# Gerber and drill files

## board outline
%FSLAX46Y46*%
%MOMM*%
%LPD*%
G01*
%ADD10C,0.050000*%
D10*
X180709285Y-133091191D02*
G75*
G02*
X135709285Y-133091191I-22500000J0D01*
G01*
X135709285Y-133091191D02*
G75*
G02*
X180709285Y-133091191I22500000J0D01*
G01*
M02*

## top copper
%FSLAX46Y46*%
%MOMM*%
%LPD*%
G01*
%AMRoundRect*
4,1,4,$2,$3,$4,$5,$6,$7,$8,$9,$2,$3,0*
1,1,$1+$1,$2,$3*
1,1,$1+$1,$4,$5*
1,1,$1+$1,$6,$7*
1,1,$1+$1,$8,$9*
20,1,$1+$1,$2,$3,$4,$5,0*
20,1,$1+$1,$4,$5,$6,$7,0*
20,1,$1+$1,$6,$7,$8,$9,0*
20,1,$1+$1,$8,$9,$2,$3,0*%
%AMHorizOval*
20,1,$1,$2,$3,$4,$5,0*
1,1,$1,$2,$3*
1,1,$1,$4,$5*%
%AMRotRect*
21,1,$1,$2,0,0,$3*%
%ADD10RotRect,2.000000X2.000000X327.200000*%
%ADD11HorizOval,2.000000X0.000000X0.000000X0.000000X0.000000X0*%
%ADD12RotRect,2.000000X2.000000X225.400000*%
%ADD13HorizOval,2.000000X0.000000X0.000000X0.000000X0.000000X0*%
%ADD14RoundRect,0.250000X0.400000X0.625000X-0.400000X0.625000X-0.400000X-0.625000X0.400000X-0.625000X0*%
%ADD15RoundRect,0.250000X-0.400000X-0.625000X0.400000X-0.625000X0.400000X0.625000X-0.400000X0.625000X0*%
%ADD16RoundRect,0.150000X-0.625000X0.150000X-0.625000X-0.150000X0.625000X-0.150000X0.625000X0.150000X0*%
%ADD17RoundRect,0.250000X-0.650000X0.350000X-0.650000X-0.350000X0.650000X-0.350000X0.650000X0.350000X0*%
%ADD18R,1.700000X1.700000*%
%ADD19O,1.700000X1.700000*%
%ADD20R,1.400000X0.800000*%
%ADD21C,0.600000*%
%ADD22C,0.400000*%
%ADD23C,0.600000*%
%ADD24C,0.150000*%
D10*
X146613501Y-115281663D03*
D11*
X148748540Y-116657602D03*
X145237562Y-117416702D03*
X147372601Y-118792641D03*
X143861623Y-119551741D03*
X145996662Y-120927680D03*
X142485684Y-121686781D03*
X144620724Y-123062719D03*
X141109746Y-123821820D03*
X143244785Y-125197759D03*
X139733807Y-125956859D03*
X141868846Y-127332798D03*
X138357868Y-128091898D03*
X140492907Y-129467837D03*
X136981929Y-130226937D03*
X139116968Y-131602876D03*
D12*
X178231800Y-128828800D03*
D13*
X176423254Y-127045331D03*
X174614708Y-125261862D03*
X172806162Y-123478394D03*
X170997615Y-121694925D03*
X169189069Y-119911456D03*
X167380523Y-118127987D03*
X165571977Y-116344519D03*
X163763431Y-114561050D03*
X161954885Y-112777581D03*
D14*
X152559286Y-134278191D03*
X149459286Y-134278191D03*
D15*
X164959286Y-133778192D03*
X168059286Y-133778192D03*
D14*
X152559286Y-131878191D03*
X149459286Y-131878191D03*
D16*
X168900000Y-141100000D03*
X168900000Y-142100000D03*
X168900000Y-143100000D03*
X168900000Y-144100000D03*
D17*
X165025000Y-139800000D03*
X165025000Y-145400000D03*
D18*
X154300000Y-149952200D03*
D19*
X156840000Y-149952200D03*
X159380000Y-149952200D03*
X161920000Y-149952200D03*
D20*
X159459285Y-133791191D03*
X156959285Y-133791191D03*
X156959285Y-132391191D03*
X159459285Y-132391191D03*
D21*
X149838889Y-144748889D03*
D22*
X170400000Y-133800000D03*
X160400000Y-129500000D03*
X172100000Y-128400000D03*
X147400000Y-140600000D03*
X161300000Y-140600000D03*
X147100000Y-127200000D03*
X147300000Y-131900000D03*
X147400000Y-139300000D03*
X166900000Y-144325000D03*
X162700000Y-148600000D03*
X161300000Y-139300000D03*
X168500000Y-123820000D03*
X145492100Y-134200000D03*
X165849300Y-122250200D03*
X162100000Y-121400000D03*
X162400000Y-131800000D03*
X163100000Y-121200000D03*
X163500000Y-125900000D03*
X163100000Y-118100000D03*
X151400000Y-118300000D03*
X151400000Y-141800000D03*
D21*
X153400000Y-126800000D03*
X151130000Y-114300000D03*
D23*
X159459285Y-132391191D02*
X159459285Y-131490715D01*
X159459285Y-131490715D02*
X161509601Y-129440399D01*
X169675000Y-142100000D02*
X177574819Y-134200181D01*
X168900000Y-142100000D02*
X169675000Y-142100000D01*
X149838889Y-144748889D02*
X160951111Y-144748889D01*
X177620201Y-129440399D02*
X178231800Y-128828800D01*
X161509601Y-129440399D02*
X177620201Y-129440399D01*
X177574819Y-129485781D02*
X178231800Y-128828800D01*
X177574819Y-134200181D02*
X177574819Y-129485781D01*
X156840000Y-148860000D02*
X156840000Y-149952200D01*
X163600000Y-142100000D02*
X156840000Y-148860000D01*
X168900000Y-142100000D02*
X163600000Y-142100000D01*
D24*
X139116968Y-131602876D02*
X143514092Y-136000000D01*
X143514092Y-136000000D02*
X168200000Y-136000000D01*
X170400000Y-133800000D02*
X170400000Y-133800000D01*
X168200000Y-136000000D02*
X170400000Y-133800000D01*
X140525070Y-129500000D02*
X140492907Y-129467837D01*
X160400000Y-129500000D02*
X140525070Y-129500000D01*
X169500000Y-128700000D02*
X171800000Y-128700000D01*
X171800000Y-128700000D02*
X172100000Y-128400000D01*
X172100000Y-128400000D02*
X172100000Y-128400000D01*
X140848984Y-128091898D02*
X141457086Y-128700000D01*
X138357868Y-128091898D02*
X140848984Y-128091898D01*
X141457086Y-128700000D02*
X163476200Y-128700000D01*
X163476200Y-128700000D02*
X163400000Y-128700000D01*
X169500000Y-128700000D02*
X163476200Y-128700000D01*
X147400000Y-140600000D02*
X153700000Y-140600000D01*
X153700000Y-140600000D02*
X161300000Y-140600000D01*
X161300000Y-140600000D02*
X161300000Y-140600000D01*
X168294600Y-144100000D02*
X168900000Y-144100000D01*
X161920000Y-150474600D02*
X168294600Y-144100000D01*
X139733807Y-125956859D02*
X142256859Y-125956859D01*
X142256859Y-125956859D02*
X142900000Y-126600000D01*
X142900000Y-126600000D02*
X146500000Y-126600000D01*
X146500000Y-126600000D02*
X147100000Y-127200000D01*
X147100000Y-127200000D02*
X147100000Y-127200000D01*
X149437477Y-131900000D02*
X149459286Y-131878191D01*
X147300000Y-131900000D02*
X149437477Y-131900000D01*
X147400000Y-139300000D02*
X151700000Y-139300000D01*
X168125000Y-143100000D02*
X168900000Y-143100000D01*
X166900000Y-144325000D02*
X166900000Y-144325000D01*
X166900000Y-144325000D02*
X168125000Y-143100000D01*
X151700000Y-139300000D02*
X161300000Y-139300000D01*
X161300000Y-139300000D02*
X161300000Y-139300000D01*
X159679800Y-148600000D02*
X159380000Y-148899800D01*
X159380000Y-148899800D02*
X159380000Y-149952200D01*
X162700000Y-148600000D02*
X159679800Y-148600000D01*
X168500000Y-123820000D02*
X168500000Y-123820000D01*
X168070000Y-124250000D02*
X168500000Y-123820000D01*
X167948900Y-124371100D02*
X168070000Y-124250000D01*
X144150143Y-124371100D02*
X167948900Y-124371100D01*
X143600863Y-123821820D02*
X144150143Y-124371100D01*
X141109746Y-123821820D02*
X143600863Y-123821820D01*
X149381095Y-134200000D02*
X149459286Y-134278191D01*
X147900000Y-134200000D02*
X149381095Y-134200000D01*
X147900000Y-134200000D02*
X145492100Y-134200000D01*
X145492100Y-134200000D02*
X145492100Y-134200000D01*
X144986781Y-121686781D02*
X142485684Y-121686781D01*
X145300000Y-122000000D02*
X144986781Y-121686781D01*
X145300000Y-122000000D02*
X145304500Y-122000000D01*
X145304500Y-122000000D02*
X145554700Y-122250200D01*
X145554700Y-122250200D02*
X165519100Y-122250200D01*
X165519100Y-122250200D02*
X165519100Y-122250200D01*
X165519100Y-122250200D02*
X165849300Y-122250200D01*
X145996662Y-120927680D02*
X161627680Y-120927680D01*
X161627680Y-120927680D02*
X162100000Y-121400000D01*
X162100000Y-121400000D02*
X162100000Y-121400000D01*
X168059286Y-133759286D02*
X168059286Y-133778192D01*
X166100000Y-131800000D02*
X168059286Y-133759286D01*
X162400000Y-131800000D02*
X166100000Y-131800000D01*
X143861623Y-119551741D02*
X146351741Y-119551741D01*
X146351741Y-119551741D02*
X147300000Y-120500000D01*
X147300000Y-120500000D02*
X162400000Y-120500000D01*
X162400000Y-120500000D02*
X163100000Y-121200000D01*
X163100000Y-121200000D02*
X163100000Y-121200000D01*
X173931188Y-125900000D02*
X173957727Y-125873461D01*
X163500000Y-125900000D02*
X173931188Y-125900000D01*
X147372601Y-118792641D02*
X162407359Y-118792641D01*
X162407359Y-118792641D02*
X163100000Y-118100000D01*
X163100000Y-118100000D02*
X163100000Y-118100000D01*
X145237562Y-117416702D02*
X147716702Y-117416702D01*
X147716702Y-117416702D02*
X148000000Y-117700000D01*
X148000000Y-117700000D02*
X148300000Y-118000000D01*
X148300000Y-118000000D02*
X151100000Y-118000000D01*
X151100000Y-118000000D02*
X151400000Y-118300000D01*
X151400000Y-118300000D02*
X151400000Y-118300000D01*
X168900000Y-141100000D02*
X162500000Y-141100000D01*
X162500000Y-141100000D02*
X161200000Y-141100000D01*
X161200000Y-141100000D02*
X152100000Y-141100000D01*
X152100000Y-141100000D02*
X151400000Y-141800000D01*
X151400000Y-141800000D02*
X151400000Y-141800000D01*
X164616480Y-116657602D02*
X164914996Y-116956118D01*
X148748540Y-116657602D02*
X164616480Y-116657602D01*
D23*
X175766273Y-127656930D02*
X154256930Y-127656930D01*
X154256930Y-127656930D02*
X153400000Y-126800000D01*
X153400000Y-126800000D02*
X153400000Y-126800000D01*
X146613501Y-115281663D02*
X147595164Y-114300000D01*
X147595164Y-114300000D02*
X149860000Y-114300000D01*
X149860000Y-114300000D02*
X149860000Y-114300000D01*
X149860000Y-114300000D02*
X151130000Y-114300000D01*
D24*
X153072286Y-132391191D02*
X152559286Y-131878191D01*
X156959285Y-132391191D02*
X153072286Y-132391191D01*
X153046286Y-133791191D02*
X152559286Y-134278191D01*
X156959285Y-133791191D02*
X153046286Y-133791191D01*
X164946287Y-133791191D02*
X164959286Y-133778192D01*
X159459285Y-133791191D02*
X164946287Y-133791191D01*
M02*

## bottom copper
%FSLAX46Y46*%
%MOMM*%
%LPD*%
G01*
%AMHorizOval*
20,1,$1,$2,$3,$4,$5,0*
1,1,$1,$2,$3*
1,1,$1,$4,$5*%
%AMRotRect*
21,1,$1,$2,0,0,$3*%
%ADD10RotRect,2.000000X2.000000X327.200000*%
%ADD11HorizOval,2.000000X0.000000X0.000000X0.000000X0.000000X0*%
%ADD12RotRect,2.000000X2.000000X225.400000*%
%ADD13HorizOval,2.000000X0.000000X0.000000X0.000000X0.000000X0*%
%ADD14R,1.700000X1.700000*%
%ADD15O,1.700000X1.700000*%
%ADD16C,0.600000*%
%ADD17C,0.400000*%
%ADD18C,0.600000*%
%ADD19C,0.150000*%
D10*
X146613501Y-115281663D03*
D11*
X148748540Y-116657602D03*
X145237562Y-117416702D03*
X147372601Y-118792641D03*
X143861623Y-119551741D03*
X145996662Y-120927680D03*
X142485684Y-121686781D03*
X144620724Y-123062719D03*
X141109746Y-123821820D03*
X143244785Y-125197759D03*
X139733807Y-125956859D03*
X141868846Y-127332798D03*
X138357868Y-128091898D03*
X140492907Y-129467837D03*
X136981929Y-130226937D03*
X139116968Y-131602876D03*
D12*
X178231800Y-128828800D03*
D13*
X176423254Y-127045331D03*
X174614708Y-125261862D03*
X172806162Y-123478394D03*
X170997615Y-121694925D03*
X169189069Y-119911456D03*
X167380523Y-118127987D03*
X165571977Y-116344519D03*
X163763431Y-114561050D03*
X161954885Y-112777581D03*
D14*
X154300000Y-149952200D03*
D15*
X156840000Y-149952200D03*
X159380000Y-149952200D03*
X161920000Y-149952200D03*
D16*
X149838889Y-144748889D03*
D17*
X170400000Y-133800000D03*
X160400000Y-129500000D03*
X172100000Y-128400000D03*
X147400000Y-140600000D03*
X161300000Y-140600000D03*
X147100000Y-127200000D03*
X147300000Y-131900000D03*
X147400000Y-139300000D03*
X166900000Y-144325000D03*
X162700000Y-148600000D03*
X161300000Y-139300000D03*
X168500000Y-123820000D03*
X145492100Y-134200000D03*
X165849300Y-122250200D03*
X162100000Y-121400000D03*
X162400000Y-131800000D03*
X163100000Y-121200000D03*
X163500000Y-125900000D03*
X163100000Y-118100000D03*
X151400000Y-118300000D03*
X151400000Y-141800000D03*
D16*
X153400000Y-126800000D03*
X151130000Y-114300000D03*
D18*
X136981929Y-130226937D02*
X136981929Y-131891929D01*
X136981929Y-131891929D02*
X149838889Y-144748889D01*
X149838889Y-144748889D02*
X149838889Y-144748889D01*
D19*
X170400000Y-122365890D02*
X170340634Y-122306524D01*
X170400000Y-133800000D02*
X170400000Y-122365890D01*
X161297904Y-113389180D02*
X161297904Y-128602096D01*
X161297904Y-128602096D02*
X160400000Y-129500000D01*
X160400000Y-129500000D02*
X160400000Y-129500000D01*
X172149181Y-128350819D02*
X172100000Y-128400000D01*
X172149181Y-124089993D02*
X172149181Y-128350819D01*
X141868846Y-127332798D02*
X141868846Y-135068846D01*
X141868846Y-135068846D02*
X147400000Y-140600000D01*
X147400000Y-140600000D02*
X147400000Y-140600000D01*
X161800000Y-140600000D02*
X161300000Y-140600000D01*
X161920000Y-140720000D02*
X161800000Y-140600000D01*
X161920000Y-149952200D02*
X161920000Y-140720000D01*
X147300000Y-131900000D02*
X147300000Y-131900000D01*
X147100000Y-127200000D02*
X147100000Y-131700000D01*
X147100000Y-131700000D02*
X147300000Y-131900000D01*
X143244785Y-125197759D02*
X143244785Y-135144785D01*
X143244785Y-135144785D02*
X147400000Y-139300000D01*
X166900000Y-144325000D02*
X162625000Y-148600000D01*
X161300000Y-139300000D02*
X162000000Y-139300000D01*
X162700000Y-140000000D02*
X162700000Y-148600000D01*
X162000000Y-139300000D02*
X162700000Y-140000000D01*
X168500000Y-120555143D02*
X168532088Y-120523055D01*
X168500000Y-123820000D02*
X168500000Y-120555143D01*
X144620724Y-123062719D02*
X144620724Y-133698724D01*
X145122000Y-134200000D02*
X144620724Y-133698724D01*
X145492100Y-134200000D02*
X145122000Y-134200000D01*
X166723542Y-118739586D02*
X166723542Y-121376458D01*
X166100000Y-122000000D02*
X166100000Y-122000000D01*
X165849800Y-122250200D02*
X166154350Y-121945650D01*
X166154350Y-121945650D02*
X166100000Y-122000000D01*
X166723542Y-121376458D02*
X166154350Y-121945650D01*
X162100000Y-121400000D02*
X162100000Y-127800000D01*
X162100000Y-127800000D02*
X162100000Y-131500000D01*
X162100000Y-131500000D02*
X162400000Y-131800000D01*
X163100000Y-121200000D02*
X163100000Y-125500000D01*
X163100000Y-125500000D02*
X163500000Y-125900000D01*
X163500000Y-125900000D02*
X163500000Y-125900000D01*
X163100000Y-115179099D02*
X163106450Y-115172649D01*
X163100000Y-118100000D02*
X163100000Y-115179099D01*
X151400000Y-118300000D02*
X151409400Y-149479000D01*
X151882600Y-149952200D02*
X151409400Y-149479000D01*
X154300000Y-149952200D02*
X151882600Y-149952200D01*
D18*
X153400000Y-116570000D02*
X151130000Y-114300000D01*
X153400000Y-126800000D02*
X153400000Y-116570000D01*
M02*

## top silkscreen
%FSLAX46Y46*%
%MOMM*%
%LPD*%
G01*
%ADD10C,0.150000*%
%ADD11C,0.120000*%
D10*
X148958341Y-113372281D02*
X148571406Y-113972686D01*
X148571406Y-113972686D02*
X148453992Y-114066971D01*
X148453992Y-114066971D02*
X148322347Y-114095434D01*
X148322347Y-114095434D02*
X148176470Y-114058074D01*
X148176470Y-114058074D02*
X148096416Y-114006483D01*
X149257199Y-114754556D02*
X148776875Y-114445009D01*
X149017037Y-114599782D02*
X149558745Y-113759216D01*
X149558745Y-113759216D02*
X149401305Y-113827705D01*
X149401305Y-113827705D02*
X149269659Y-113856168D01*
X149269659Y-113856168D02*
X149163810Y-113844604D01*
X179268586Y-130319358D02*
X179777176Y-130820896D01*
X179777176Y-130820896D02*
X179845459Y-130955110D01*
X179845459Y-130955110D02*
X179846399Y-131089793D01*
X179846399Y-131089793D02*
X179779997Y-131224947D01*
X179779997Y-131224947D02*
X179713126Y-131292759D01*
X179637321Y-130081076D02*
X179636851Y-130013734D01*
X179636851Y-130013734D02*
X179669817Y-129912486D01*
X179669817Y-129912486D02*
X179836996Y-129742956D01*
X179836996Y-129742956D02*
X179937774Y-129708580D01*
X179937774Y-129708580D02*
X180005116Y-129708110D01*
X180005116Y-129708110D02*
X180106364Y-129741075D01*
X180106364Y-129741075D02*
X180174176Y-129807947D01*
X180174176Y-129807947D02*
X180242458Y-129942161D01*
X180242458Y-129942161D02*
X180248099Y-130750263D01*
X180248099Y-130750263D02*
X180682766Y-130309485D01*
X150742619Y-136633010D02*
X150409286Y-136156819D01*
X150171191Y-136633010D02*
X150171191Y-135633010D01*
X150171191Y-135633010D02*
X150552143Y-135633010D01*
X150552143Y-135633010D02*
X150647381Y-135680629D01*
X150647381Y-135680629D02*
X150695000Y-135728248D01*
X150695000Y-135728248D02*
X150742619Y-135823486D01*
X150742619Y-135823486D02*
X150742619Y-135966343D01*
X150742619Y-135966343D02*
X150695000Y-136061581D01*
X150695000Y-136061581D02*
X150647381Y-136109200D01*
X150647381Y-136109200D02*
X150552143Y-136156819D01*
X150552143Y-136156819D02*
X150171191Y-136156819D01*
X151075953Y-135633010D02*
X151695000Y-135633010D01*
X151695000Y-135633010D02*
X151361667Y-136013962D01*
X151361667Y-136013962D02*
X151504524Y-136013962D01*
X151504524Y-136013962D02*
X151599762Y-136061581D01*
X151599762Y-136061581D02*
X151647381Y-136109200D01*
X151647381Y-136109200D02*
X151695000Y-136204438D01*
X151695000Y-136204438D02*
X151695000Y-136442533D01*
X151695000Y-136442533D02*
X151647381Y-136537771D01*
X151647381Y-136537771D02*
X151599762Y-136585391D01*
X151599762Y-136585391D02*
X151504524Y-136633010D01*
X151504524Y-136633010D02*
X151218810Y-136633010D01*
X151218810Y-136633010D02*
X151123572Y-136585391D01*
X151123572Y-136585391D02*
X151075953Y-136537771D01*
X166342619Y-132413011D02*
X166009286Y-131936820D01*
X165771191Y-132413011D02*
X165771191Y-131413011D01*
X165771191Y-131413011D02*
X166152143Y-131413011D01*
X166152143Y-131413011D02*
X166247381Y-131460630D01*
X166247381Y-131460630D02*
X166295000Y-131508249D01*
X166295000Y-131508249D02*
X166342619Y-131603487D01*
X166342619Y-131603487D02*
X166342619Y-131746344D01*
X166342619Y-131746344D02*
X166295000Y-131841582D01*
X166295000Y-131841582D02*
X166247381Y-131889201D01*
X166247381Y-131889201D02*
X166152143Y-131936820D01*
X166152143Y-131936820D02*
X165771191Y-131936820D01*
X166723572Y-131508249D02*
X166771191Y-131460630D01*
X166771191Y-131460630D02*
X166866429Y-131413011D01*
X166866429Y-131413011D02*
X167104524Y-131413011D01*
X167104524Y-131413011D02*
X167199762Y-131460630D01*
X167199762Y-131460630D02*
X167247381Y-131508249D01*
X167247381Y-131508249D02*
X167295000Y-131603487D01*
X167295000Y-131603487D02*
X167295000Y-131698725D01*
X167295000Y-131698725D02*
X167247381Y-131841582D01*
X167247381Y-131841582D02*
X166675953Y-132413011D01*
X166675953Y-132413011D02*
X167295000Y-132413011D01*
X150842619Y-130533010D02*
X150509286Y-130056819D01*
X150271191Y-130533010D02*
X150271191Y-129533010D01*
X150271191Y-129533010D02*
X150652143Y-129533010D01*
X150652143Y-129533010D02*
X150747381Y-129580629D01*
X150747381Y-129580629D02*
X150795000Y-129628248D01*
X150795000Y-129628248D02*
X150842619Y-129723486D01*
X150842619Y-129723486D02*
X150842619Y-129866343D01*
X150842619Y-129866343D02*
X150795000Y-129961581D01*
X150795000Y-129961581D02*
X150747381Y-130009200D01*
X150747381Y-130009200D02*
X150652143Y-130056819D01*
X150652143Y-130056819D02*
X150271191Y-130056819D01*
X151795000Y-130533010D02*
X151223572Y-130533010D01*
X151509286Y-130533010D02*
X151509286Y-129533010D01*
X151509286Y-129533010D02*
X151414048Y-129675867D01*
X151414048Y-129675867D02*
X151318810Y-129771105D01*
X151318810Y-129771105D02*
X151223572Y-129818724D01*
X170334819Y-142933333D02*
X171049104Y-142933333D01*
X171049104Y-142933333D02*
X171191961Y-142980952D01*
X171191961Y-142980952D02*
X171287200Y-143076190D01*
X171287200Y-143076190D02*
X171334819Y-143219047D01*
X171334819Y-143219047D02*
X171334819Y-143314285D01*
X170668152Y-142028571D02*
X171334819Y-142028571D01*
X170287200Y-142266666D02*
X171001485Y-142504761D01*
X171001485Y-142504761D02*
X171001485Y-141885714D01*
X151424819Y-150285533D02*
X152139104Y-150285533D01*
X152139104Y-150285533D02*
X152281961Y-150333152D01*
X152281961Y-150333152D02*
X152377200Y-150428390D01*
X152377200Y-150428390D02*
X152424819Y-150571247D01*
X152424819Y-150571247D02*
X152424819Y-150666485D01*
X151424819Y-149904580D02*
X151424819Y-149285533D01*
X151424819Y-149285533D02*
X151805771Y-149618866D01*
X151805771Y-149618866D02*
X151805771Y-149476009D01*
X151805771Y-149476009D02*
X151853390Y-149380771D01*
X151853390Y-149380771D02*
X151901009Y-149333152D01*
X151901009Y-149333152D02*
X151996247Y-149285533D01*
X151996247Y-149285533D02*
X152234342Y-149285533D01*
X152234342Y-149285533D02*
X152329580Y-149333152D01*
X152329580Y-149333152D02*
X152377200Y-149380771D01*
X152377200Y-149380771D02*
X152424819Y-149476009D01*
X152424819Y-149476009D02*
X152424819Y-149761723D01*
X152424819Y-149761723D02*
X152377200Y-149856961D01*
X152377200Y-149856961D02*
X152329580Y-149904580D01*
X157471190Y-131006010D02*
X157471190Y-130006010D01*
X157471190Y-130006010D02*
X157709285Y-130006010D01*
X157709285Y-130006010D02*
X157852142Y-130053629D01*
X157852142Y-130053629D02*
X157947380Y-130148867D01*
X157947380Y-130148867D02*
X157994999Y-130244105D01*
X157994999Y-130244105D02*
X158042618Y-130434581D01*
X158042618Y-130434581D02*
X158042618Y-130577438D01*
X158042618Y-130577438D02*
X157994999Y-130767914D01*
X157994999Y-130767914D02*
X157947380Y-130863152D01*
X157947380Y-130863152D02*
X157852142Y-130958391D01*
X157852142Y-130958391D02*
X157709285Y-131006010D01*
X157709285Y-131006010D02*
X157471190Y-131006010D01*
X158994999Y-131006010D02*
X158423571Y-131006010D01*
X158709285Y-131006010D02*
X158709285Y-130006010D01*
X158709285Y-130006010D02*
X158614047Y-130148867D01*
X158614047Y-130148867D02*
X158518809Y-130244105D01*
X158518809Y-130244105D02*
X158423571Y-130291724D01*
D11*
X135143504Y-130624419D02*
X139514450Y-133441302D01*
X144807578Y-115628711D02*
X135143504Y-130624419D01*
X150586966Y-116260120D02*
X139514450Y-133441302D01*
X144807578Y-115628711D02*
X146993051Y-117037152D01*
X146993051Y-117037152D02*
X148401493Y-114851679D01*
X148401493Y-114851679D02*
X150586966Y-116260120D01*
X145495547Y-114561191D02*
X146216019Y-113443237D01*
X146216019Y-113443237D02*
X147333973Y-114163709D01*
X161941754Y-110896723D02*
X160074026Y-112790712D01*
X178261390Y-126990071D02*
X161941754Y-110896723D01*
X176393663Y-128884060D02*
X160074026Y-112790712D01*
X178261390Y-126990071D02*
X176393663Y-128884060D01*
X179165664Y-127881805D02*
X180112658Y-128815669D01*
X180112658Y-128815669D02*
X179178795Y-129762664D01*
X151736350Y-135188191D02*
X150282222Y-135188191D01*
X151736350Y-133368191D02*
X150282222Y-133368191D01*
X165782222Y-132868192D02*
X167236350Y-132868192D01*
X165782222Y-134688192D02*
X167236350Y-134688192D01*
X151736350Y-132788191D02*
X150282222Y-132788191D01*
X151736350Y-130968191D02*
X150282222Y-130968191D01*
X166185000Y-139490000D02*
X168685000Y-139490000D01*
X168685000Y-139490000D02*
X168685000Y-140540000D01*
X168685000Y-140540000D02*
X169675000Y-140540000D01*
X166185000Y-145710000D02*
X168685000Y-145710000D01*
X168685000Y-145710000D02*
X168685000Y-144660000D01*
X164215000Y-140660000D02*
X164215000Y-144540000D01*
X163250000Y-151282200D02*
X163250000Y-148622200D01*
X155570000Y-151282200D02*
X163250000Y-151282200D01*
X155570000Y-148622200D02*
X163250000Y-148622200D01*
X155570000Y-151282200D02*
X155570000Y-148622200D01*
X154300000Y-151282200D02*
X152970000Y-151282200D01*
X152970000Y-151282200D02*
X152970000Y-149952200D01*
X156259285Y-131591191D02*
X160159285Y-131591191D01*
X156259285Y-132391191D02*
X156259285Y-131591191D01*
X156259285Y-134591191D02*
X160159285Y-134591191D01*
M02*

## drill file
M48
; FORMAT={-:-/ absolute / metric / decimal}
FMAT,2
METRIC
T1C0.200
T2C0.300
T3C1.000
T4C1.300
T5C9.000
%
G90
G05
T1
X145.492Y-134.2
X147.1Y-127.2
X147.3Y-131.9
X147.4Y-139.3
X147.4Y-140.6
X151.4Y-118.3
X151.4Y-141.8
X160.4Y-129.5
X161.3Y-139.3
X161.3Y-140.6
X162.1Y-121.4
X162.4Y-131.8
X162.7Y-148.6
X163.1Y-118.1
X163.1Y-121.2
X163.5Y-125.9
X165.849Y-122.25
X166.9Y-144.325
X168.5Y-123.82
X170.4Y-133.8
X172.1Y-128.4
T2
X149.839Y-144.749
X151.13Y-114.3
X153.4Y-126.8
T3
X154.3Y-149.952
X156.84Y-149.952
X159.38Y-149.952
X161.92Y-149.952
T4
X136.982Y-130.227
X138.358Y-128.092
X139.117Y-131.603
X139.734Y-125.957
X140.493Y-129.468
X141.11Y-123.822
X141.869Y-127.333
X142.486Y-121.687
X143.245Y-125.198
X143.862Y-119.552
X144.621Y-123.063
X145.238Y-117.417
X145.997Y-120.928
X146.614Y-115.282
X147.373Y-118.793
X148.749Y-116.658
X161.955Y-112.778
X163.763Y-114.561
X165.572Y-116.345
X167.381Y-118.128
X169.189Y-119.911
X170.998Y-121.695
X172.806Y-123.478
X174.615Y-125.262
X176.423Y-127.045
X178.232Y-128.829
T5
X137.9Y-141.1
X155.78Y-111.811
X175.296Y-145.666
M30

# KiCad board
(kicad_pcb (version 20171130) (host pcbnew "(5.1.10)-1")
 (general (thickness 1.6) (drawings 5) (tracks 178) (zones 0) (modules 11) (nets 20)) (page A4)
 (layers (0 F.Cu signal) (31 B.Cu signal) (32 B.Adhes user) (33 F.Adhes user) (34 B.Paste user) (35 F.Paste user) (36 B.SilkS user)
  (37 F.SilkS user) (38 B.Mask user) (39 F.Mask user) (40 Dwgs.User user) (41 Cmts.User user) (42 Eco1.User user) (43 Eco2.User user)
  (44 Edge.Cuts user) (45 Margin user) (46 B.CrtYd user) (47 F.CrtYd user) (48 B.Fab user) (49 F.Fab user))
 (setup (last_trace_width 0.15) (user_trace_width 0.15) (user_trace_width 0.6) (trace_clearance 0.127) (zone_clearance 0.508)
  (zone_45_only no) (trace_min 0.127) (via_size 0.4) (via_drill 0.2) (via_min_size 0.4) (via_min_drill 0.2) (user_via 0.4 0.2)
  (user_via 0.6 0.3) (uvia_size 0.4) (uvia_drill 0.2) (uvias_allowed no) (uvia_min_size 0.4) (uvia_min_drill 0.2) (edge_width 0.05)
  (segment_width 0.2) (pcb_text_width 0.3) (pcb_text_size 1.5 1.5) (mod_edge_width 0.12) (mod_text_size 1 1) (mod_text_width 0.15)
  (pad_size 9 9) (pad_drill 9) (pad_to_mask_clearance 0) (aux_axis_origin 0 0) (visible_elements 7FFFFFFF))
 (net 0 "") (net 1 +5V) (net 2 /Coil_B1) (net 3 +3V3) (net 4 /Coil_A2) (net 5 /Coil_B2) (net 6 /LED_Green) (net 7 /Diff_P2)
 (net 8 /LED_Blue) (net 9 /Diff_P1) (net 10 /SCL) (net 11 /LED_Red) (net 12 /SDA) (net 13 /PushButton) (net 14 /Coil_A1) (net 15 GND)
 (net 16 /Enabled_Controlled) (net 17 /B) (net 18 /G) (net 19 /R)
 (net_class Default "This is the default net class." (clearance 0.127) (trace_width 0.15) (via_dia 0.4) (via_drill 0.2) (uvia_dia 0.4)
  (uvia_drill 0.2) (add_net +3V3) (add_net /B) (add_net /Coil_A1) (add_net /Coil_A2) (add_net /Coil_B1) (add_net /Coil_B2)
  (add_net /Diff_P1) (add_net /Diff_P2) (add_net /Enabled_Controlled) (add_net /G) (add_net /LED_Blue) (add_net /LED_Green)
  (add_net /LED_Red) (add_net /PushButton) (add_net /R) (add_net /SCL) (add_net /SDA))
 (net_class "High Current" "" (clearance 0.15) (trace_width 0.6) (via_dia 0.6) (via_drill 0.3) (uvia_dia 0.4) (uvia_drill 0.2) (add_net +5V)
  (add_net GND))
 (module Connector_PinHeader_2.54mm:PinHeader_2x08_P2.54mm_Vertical (layer F.Cu) (at 146.613501 115.281663 327.2)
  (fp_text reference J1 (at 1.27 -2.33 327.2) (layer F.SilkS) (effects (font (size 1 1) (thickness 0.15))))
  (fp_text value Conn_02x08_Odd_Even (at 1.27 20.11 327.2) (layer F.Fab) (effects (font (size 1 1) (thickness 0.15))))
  (fp_line (start -1.33 19.11) (end 3.87 19.11) (layer F.SilkS) (width 0.12))
  (fp_line (start -1.33 1.27) (end -1.33 19.11) (layer F.SilkS) (width 0.12))
  (fp_line (start 3.87 -1.33) (end 3.87 19.11) (layer F.SilkS) (width 0.12))
  (fp_line (start -1.33 1.27) (end 1.27 1.27) (layer F.SilkS) (width 0.12))
  (fp_line (start 1.27 1.27) (end 1.27 -1.33) (layer F.SilkS) (width 0.12))
  (fp_line (start 1.27 -1.33) (end 3.87 -1.33) (layer F.SilkS) (width 0.12))
  (fp_line (start -1.33 0) (end -1.33 -1.33) (layer F.SilkS) (width 0.12))
  (fp_line (start -1.33 -1.33) (end 0 -1.33) (layer F.SilkS) (width 0.12))
  (pad 1 thru_hole rect (at 0 0 327.2) (size 2 2) (drill 1.3) (layers *.Cu *.Mask) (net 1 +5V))
  (pad 2 thru_hole oval (at 2.54 0 327.2) (size 2 2) (drill 1.3) (layers *.Cu *.Mask) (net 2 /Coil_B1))
  (pad 3 thru_hole oval (at 0 2.54 327.2) (size 2 2) (drill 1.3) (layers *.Cu *.Mask) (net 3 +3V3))
  (pad 4 thru_hole oval (at 2.54 2.54 327.2) (size 2 2) (drill 1.3) (layers *.Cu *.Mask) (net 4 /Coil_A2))
  (pad 5 thru_hole oval (at 0 5.08 327.2) (size 2 2) (drill 1.3) (layers *.Cu *.Mask) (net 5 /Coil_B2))
  (pad 6 thru_hole oval (at 2.54 5.08 327.2) (size 2 2) (drill 1.3) (layers *.Cu *.Mask) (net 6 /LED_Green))
  (pad 7 thru_hole oval (at 0 7.620001 327.2) (size 2 2) (drill 1.3) (layers *.Cu *.Mask) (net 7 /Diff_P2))
  (pad 8 thru_hole oval (at 2.54 7.619999 327.2) (size 2 2) (drill 1.3) (layers *.Cu *.Mask) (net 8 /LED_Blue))
  (pad 9 thru_hole oval (at 0.000001 10.16 327.2) (size 2 2) (drill 1.3) (layers *.Cu *.Mask) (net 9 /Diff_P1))
  (pad 10 thru_hole oval (at 2.54 10.16 327.2) (size 2 2) (drill 1.3) (layers *.Cu *.Mask) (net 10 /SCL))
  (pad 11 thru_hole oval (at 0 12.7 327.2) (size 2 2) (drill 1.3) (layers *.Cu *.Mask) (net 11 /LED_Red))
  (pad 12 thru_hole oval (at 2.54 12.7 327.2) (size 2 2) (drill 1.3) (layers *.Cu *.Mask) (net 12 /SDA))
  (pad 13 thru_hole oval (at 0 15.24 327.2) (size 2 2) (drill 1.3) (layers *.Cu *.Mask) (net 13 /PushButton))
  (pad 14 thru_hole oval (at 2.54 15.24 327.2) (size 2 2) (drill 1.3) (layers *.Cu *.Mask) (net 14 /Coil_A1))
  (pad 15 thru_hole oval (at 0 17.78 327.2) (size 2 2) (drill 1.3) (layers *.Cu *.Mask) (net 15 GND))
  (pad 16 thru_hole oval (at 2.54 17.78 327.2) (size 2 2) (drill 1.3) (layers *.Cu *.Mask) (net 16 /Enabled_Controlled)))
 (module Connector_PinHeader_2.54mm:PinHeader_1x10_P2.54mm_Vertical (layer F.Cu) (at 178.2318 128.8288 225.4)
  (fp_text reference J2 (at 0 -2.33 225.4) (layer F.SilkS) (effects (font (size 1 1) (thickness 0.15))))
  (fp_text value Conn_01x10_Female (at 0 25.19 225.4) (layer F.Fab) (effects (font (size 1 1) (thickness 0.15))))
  (fp_line (start -1.33 24.19) (end 1.33 24.19) (layer F.SilkS) (width 0.12))
  (fp_line (start -1.33 1.27) (end -1.33 24.19) (layer F.SilkS) (width 0.12))
  (fp_line (start 1.33 1.27) (end 1.33 24.19) (layer F.SilkS) (width 0.12))
  (fp_line (start -1.33 1.27) (end 1.33 1.27) (layer F.SilkS) (width 0.12))
  (fp_line (start -1.33 0) (end -1.33 -1.33) (layer F.SilkS) (width 0.12))
  (fp_line (start -1.33 -1.33) (end 0 -1.33) (layer F.SilkS) (width 0.12))
  (pad 1 thru_hole rect (at 0 0 225.4) (size 2 2) (drill 1.3) (layers *.Cu *.Mask) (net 15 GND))
  (pad 2 thru_hole oval (at 0 2.54 225.4) (size 2 2) (drill 1.3) (layers *.Cu *.Mask) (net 1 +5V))
  (pad 3 thru_hole oval (at -0.000001 5.08 225.4) (size 2 2) (drill 1.3) (layers *.Cu *.Mask) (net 5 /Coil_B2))
  (pad 4 thru_hole oval (at 0 7.619999 225.4) (size 2 2) (drill 1.3) (layers *.Cu *.Mask) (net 13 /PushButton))
  (pad 5 thru_hole oval (at 0 10.16 225.4) (size 2 2) (drill 1.3) (layers *.Cu *.Mask) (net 16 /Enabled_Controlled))
  (pad 6 thru_hole oval (at 0 12.7 225.4) (size 2 2) (drill 1.3) (layers *.Cu *.Mask) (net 9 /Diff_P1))
  (pad 7 thru_hole oval (at 0 15.24 225.4) (size 2 2) (drill 1.3) (layers *.Cu *.Mask) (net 7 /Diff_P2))
  (pad 8 thru_hole oval (at 0 17.78 225.4) (size 2 2) (drill 1.3) (layers *.Cu *.Mask) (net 2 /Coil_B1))
  (pad 9 thru_hole oval (at 0 20.32 225.4) (size 2 2) (drill 1.3) (layers *.Cu *.Mask) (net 4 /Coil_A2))
  (pad 10 thru_hole oval (at 0 22.86 225.4) (size 2 2) (drill 1.3) (layers *.Cu *.Mask) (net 14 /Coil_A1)))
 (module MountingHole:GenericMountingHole (layer F.Cu) (at 175.295814 145.666378 45)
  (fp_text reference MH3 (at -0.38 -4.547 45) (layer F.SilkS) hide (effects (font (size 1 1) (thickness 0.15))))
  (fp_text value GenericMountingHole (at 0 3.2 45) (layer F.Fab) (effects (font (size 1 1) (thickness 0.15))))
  (pad "" np_thru_hole circle (at 0 0 45) (size 9 9) (drill 9) (layers *.Cu *.Mask)))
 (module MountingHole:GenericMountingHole (layer F.Cu) (at 137.9 141.1 45)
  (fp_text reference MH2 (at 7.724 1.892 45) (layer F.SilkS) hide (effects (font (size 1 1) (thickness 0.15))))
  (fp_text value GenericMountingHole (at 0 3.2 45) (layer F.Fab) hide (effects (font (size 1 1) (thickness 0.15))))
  (pad "" np_thru_hole circle (at 0 0 45) (size 9 9) (drill 9) (layers *.Cu *.Mask)))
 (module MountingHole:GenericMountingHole (layer F.Cu) (at 155.780374 111.810813 45)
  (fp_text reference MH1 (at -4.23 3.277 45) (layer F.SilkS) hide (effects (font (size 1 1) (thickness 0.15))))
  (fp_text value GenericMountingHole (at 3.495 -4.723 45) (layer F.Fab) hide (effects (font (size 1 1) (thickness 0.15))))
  (pad "" np_thru_hole circle (at 0 0 45) (size 9 9) (drill 9) (layers *.Cu *.Mask)))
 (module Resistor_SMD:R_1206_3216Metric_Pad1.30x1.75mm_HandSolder (layer F.Cu) (at 151.009286 134.278191 180)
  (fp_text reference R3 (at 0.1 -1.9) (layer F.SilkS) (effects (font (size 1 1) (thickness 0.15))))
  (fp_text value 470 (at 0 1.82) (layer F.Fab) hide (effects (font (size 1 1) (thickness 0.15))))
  (fp_line (start -0.727064 -0.91) (end 0.727064 -0.91) (layer F.SilkS) (width 0.12))
  (fp_line (start -0.727064 0.91) (end 0.727064 0.91) (layer F.SilkS) (width 0.12))
  (pad 1 smd roundrect (at -1.55 0 180) (size 1.3 1.75) (layers F.Cu F.Paste F.Mask) (roundrect_rratio 0.192308) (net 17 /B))
  (pad 2 smd roundrect (at 1.55 0 180) (size 1.3 1.75) (layers F.Cu F.Paste F.Mask) (roundrect_rratio 0.192308) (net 8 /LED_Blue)))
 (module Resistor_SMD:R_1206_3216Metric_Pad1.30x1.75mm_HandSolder (layer F.Cu) (at 166.509286 133.778192)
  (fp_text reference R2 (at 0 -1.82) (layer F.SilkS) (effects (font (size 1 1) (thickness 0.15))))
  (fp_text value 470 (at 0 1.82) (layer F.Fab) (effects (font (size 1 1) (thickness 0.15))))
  (fp_line (start -0.727064 -0.91) (end 0.727064 -0.91) (layer F.SilkS) (width 0.12))
  (fp_line (start -0.727064 0.91) (end 0.727064 0.91) (layer F.SilkS) (width 0.12))
  (pad 1 smd roundrect (at -1.55 0) (size 1.3 1.75) (layers F.Cu F.Paste F.Mask) (roundrect_rratio 0.192308) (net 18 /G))
  (pad 2 smd roundrect (at 1.55 0) (size 1.3 1.75) (layers F.Cu F.Paste F.Mask) (roundrect_rratio 0.192308) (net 6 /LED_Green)))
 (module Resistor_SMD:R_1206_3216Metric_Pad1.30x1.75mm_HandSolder (layer F.Cu) (at 151.009286 131.878191 180)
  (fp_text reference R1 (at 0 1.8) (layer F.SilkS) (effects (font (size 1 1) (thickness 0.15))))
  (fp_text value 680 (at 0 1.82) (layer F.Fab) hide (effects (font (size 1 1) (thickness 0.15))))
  (fp_line (start -0.727064 -0.91) (end 0.727064 -0.91) (layer F.SilkS) (width 0.12))
  (fp_line (start -0.727064 0.91) (end 0.727064 0.91) (layer F.SilkS) (width 0.12))
  (pad 1 smd roundrect (at -1.55 0 180) (size 1.3 1.75) (layers F.Cu F.Paste F.Mask) (roundrect_rratio 0.192308) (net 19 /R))
  (pad 2 smd roundrect (at 1.55 0 180) (size 1.3 1.75) (layers F.Cu F.Paste F.Mask) (roundrect_rratio 0.192308) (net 11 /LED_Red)))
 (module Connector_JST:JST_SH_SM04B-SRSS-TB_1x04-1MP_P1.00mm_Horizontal (layer F.Cu) (at 166.9 142.6 270)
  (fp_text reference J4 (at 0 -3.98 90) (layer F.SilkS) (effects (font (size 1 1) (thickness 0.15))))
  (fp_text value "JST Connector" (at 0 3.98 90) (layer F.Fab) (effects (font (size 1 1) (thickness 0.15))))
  (fp_line (start -3.11 0.715) (end -3.11 -1.785) (layer F.SilkS) (width 0.12))
  (fp_line (start -3.11 -1.785) (end -2.06 -1.785) (layer F.SilkS) (width 0.12))
  (fp_line (start -2.06 -1.785) (end -2.06 -2.775) (layer F.SilkS) (width 0.12))
  (fp_line (start 3.11 0.715) (end 3.11 -1.785) (layer F.SilkS) (width 0.12))
  (fp_line (start 3.11 -1.785) (end 2.06 -1.785) (layer F.SilkS) (width 0.12))
  (fp_line (start -1.94 2.685) (end 1.94 2.685) (layer F.SilkS) (width 0.12))
  (pad 1 smd roundrect (at -1.5 -2 270) (size 0.6 1.55) (layers F.Cu F.Paste F.Mask) (roundrect_rratio 0.25) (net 3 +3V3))
  (pad 2 smd roundrect (at -0.5 -2 270) (size 0.6 1.55) (layers F.Cu F.Paste F.Mask) (roundrect_rratio 0.25) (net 15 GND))
  (pad 3 smd roundrect (at 0.5 -2 270) (size 0.6 1.55) (layers F.Cu F.Paste F.Mask) (roundrect_rratio 0.25) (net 10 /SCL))
  (pad 4 smd roundrect (at 1.5 -2 270) (size 0.6 1.55) (layers F.Cu F.Paste F.Mask) (roundrect_rratio 0.25) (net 12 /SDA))
  (pad MP smd roundrect (at -2.8 1.875 270) (size 1.2 1.8) (layers F.Cu F.Paste F.Mask) (roundrect_rratio 0.208333))
  (pad MP smd roundrect (at 2.8 1.875 270) (size 1.2 1.8) (layers F.Cu F.Paste F.Mask) (roundrect_rratio 0.208333)))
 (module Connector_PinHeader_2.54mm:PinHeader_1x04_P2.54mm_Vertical (layer F.Cu) (at 154.3 149.9522 90)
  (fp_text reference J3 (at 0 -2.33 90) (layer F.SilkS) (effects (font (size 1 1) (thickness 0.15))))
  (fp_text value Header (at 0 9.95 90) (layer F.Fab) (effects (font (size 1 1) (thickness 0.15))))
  (fp_line (start -1.33 8.95) (end 1.33 8.95) (layer F.SilkS) (width 0.12))
  (fp_line (start -1.33 1.27) (end -1.33 8.95) (layer F.SilkS) (width 0.12))
  (fp_line (start 1.33 1.27) (end 1.33 8.95) (layer F.SilkS) (width 0.12))
  (fp_line (start -1.33 1.27) (end 1.33 1.27) (layer F.SilkS) (width 0.12))
  (fp_line (start -1.33 0) (end -1.33 -1.33) (layer F.SilkS) (width 0.12))
  (fp_line (start -1.33 -1.33) (end 0 -1.33) (layer F.SilkS) (width 0.12))
  (pad 1 thru_hole rect (at 0 0 90) (size 1.7 1.7) (drill 1) (layers *.Cu *.Mask) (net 3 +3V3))
  (pad 2 thru_hole oval (at 0 2.54 90) (size 1.7 1.7) (drill 1) (layers *.Cu *.Mask) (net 15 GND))
  (pad 3 thru_hole oval (at 0 5.08 90) (size 1.7 1.7) (drill 1) (layers *.Cu *.Mask) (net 10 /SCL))
  (pad 4 thru_hole oval (at 0 7.62 90) (size 1.7 1.7) (drill 1) (layers *.Cu *.Mask) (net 12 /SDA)))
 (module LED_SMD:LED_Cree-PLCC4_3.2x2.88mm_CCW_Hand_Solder (layer F.Cu) (at 158.209285 133.091191)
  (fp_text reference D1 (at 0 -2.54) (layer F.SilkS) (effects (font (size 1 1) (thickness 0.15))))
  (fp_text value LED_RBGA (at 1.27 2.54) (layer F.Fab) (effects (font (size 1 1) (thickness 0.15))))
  (fp_line (start -1.95 -1.5) (end 1.95 -1.5) (layer F.SilkS) (width 0.12))
  (fp_line (start -1.95 -0.7) (end -1.95 -1.5) (layer F.SilkS) (width 0.12))
  (fp_line (start -1.95 1.5) (end 1.95 1.5) (layer F.SilkS) (width 0.12))
  (pad 3 smd rect (at 1.25 0.7) (size 1.4 0.8) (layers F.Cu F.Paste F.Mask) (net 18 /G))
  (pad 2 smd rect (at -1.25 0.7) (size 1.4 0.8) (layers F.Cu F.Paste F.Mask) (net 17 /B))
  (pad 1 smd rect (at -1.25 -0.7) (size 1.4 0.8) (layers F.Cu F.Paste F.Mask) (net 19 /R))
  (pad 4 smd rect (at 1.25 -0.7) (size 1.4 0.8) (layers F.Cu F.Paste F.Mask) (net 15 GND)))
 (gr_circle (center 158.209285 133.091191) (end 142.299383 149.001094) (layer Edge.Cuts) (width 0.05))
 (segment (start 159.459285 132.391191) (end 159.459285 131.490715) (width 0.6) (layer F.Cu) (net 15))
 (segment (start 159.459285 131.490715) (end 161.509601 129.440399) (width 0.6) (layer F.Cu) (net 15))
 (segment (start 136.981929 130.226937) (end 136.981929 131.891929) (width 0.6) (layer B.Cu) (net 15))
 (segment (start 136.981929 131.891929) (end 149.838889 144.748889) (width 0.6) (layer B.Cu) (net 15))
 (segment (start 169.675 142.1) (end 177.574819 134.200181) (width 0.6) (layer F.Cu) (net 15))
 (segment (start 168.9 142.1) (end 169.675 142.1) (width 0.6) (layer F.Cu) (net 15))
 (segment (start 149.838889 144.748889) (end 149.838889 144.748889) (width 0.6) (layer B.Cu) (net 15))
 (via (at 149.838889 144.748889) (size 0.6) (drill 0.3) (layers F.Cu B.Cu) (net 15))
 (segment (start 149.838889 144.748889) (end 160.951111 144.748889) (width 0.6) (layer F.Cu) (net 15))
 (segment (start 177.620201 129.440399) (end 178.2318 128.8288) (width 0.6) (layer F.Cu) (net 15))
 (segment (start 161.509601 129.440399) (end 177.620201 129.440399) (width 0.6) (layer F.Cu) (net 15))
 (segment (start 177.574819 129.485781) (end 178.2318 128.8288) (width 0.6) (layer F.Cu) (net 15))
 (segment (start 177.574819 134.200181) (end 177.574819 129.485781) (width 0.6) (layer F.Cu) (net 15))
 (segment (start 156.84 148.86) (end 156.84 149.9522) (width 0.6) (layer F.Cu) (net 15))
 (segment (start 163.6 142.1) (end 156.84 148.86) (width 0.6) (layer F.Cu) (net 15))
 (segment (start 168.9 142.1) (end 163.6 142.1) (width 0.6) (layer F.Cu) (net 15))
 (segment (start 139.116968 131.602876) (end 143.514092 136) (width 0.15) (layer F.Cu) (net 16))
 (segment (start 143.514092 136) (end 168.2 136) (width 0.15) (layer F.Cu) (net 16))
 (segment (start 170.4 122.36589) (end 170.340634 122.306524) (width 0.15) (layer B.Cu) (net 16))
 (segment (start 170.4 133.8) (end 170.4 122.36589) (width 0.15) (layer B.Cu) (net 16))
 (segment (start 170.4 133.8) (end 170.4 133.8) (width 0.15) (layer F.Cu) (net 16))
 (segment (start 168.2 136) (end 170.4 133.8) (width 0.15) (layer F.Cu) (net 16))
 (via (at 170.4 133.8) (size 0.4) (drill 0.2) (layers F.Cu B.Cu) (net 16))
 (segment (start 161.297904 113.38918) (end 161.297904 128.602096) (width 0.15) (layer B.Cu) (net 14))
 (segment (start 161.297904 128.602096) (end 160.4 129.5) (width 0.15) (layer B.Cu) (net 14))
 (segment (start 160.4 129.5) (end 160.4 129.5) (width 0.15) (layer B.Cu) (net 14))
 (via (at 160.4 129.5) (size 0.4) (drill 0.2) (layers F.Cu B.Cu) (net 14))
 (segment (start 140.52507 129.5) (end 140.492907 129.467837) (width 0.15) (layer F.Cu) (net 14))
 (segment (start 160.4 129.5) (end 140.52507 129.5) (width 0.15) (layer F.Cu) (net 14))
 (segment (start 169.5 128.7) (end 171.8 128.7) (width 0.15) (layer F.Cu) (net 13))
 (segment (start 171.8 128.7) (end 172.1 128.4) (width 0.15) (layer F.Cu) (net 13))
 (segment (start 172.1 128.4) (end 172.1 128.4) (width 0.15) (layer F.Cu) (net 13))
 (via (at 172.1 128.4) (size 0.4) (drill 0.2) (layers F.Cu B.Cu) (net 13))
 (segment (start 172.149181 128.350819) (end 172.1 128.4) (width 0.15) (layer B.Cu) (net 13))
 (segment (start 172.149181 124.089993) (end 172.149181 128.350819) (width 0.15) (layer B.Cu) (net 13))
 (segment (start 140.848984 128.091898) (end 141.457086 128.7) (width 0.15) (layer F.Cu) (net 13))
 (segment (start 138.357868 128.091898) (end 140.848984 128.091898) (width 0.15) (layer F.Cu) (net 13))
 (segment (start 141.457086 128.7) (end 163.4762 128.7) (width 0.15) (layer F.Cu) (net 13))
 (segment (start 163.4762 128.7) (end 163.4 128.7) (width 0.15) (layer F.Cu) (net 13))
 (segment (start 169.5 128.7) (end 163.4762 128.7) (width 0.15) (layer F.Cu) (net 13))
 (segment (start 141.868846 127.332798) (end 141.868846 135.068846) (width 0.15) (layer B.Cu) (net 12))
 (segment (start 141.868846 135.068846) (end 147.4 140.6) (width 0.15) (layer B.Cu) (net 12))
 (segment (start 147.4 140.6) (end 147.4 140.6) (width 0.15) (layer B.Cu) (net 12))
 (via (at 147.4 140.6) (size 0.4) (drill 0.2) (layers F.Cu B.Cu) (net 12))
 (segment (start 147.4 140.6) (end 153.7 140.6) (width 0.15) (layer F.Cu) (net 12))
 (segment (start 153.7 140.6) (end 161.3 140.6) (width 0.15) (layer F.Cu) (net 12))
 (segment (start 161.3 140.6) (end 161.3 140.6) (width 0.15) (layer F.Cu) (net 12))
 (via (at 161.3 140.6) (size 0.4) (drill 0.2) (layers F.Cu B.Cu) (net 12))
 (segment (start 168.2946 144.1) (end 168.9 144.1) (width 0.15) (layer F.Cu) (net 12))
 (segment (start 161.92 150.4746) (end 168.2946 144.1) (width 0.15) (layer F.Cu) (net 12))
 (segment (start 161.8 140.6) (end 161.3 140.6) (width 0.15) (layer B.Cu) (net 12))
 (segment (start 161.92 140.72) (end 161.8 140.6) (width 0.15) (layer B.Cu) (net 12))
 (segment (start 161.92 149.9522) (end 161.92 140.72) (width 0.15) (layer B.Cu) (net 12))
 (segment (start 139.733807 125.956859) (end 142.256859 125.956859) (width 0.15) (layer F.Cu) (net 11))
 (segment (start 142.256859 125.956859) (end 142.9 126.6) (width 0.15) (layer F.Cu) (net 11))
 (segment (start 142.9 126.6) (end 146.5 126.6) (width 0.15) (layer F.Cu) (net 11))
 (segment (start 146.5 126.6) (end 147.1 127.2) (width 0.15) (layer F.Cu) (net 11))
 (segment (start 147.1 127.2) (end 147.1 127.2) (width 0.15) (layer F.Cu) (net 11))
 (via (at 147.1 127.2) (size 0.4) (drill 0.2) (layers F.Cu B.Cu) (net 11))
 (segment (start 149.437477 131.9) (end 149.459286 131.878191) (width 0.15) (layer F.Cu) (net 11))
 (segment (start 147.3 131.9) (end 147.3 131.9) (width 0.15) (layer B.Cu) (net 11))
 (segment (start 147.1 127.2) (end 147.1 131.7) (width 0.15) (layer B.Cu) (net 11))
 (segment (start 147.1 131.7) (end 147.3 131.9) (width 0.15) (layer B.Cu) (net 11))
 (via (at 147.3 131.9) (size 0.4) (drill 0.2) (layers F.Cu B.Cu) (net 11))
 (segment (start 147.3 131.9) (end 149.437477 131.9) (width 0.15) (layer F.Cu) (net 11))
 (segment (start 143.244785 125.197759) (end 143.244785 135.144785) (width 0.15) (layer B.Cu) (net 10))
 (segment (start 143.244785 135.144785) (end 147.4 139.3) (width 0.15) (layer B.Cu) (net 10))
 (via (at 147.4 139.3) (size 0.4) (drill 0.2) (layers F.Cu B.Cu) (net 10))
 (segment (start 147.4 139.3) (end 151.7 139.3) (width 0.15) (layer F.Cu) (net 10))
 (segment (start 168.125 143.1) (end 168.9 143.1) (width 0.15) (layer F.Cu) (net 10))
 (segment (start 166.9 144.325) (end 166.9 144.325) (width 0.15) (layer F.Cu) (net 10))
 (segment (start 166.9 144.325) (end 168.125 143.1) (width 0.15) (layer F.Cu) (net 10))
 (via (at 166.9 144.325) (size 0.4) (drill 0.2) (layers F.Cu B.Cu) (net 10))
 (segment (start 166.9 144.325) (end 162.625 148.6) (width 0.15) (layer B.Cu) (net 10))
 (via (at 162.7 148.6) (size 0.4) (drill 0.2) (layers F.Cu B.Cu) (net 10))
 (segment (start 151.7 139.3) (end 161.3 139.3) (width 0.15) (layer F.Cu) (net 10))
 (segment (start 161.3 139.3) (end 161.3 139.3) (width 0.15) (layer F.Cu) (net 10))
 (via (at 161.3 139.3) (size 0.4) (drill 0.2) (layers F.Cu B.Cu) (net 10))
 (segment (start 161.3 139.3) (end 162 139.3) (width 0.15) (layer B.Cu) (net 10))
 (segment (start 162.7 140) (end 162.7 148.6) (width 0.15) (layer B.Cu) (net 10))
 (segment (start 162 139.3) (end 162.7 140) (width 0.15) (layer B.Cu) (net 10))
 (segment (start 159.6798 148.6) (end 159.38 148.8998) (width 0.15) (layer F.Cu) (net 10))
 (segment (start 159.38 148.8998) (end 159.38 149.9522) (width 0.15) (layer F.Cu) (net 10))
 (segment (start 162.7 148.6) (end 159.6798 148.6) (width 0.15) (layer F.Cu) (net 10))
 (segment (start 168.5 123.82) (end 168.5 123.82) (width 0.15) (layer F.Cu) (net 9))
 (via (at 168.5 123.82) (size 0.4) (drill 0.2) (layers F.Cu B.Cu) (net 9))
 (segment (start 168.5 120.555143) (end 168.532088 120.523055) (width 0.15) (layer B.Cu) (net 9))
 (segment (start 168.5 123.82) (end 168.5 120.555143) (width 0.15) (layer B.Cu) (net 9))
 (segment (start 168.07 124.25) (end 168.5 123.82) (width 0.15) (layer F.Cu) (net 9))
 (segment (start 167.9489 124.3711) (end 168.07 124.25) (width 0.15) (layer F.Cu) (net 9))
 (segment (start 144.150143 124.3711) (end 167.9489 124.3711) (width 0.15) (layer F.Cu) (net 9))
 (segment (start 143.600863 123.82182) (end 144.150143 124.3711) (width 0.15) (layer F.Cu) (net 9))
 (segment (start 141.109746 123.82182) (end 143.600863 123.82182) (width 0.15) (layer F.Cu) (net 9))
 (segment (start 149.381095 134.2) (end 149.459286 134.278191) (width 0.15) (layer F.Cu) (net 8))
 (segment (start 147.9 134.2) (end 149.381095 134.2) (width 0.15) (layer F.Cu) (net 8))
 (segment (start 144.620724 123.062719) (end 144.620724 133.698724) (width 0.15) (layer B.Cu) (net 8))
 (segment (start 147.9 134.2) (end 145.4921 134.2) (width 0.15) (layer F.Cu) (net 8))
 (segment (start 145.4921 134.2) (end 145.4921 134.2) (width 0.15) (layer F.Cu) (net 8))
 (via (at 145.4921 134.2) (size 0.4) (drill 0.2) (layers F.Cu B.Cu) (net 8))
 (segment (start 145.122 134.2) (end 144.620724 133.698724) (width 0.15) (layer B.Cu) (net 8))
 (segment (start 145.4921 134.2) (end 145.122 134.2) (width 0.15) (layer B.Cu) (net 8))
 (segment (start 166.723542 118.739586) (end 166.723542 121.376458) (width 0.15) (layer B.Cu) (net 7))
 (segment (start 166.1 122) (end 166.1 122) (width 0.15) (layer B.Cu) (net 7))
 (segment (start 144.986781 121.686781) (end 142.485684 121.686781) (width 0.15) (layer F.Cu) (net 7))
 (segment (start 145.3 122) (end 144.986781 121.686781) (width 0.15) (layer F.Cu) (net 7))
 (segment (start 145.3 122) (end 145.3045 122) (width 0.15) (layer F.Cu) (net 7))
 (segment (start 145.3045 122) (end 145.5547 122.2502) (width 0.15) (layer F.Cu) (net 7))
 (segment (start 145.5547 122.2502) (end 165.5191 122.2502) (width 0.15) (layer F.Cu) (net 7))
 (segment (start 165.5191 122.2502) (end 165.5191 122.2502) (width 0.15) (layer F.Cu) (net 7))
 (via (at 165.8493 122.2502) (size 0.4) (drill 0.2) (layers F.Cu B.Cu) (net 7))
 (segment (start 165.8498 122.2502) (end 166.15435 121.94565) (width 0.15) (layer B.Cu) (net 7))
 (segment (start 166.15435 121.94565) (end 166.1 122) (width 0.15) (layer B.Cu) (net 7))
 (segment (start 166.723542 121.376458) (end 166.15435 121.94565) (width 0.15) (layer B.Cu) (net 7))
 (segment (start 165.5191 122.2502) (end 165.8493 122.2502) (width 0.15) (layer F.Cu) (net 7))
 (segment (start 145.996662 120.92768) (end 161.62768 120.92768) (width 0.15) (layer F.Cu) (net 6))
 (segment (start 161.62768 120.92768) (end 162.1 121.4) (width 0.15) (layer F.Cu) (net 6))
 (segment (start 162.1 121.4) (end 162.1 121.4) (width 0.15) (layer F.Cu) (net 6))
 (via (at 162.1 121.4) (size 0.4) (drill 0.2) (layers F.Cu B.Cu) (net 6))
 (segment (start 162.1 121.4) (end 162.1 127.8) (width 0.15) (layer B.Cu) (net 6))
 (via (at 162.4 131.8) (size 0.4) (drill 0.2) (layers F.Cu B.Cu) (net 6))
 (segment (start 168.059286 133.759286) (end 168.059286 133.778192) (width 0.15) (layer F.Cu) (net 6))
 (segment (start 166.1 131.8) (end 168.059286 133.759286) (width 0.15) (layer F.Cu) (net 6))
 (segment (start 162.1 127.8) (end 162.1 131.5) (width 0.15) (layer B.Cu) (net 6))
 (segment (start 162.1 131.5) (end 162.4 131.8) (width 0.15) (layer B.Cu) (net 6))
 (segment (start 162.4 131.8) (end 166.1 131.8) (width 0.15) (layer F.Cu) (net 6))
 (segment (start 143.861623 119.551741) (end 146.351741 119.551741) (width 0.15) (layer F.Cu) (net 5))
 (segment (start 146.351741 119.551741) (end 147.3 120.5) (width 0.15) (layer F.Cu) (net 5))
 (segment (start 147.3 120.5) (end 162.4 120.5) (width 0.15) (layer F.Cu) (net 5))
 (segment (start 162.4 120.5) (end 163.1 121.2) (width 0.15) (layer F.Cu) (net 5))
 (segment (start 163.1 121.2) (end 163.1 121.2) (width 0.15) (layer F.Cu) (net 5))
 (via (at 163.1 121.2) (size 0.4) (drill 0.2) (layers F.Cu B.Cu) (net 5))
 (segment (start 163.1 121.2) (end 163.1 125.5) (width 0.15) (layer B.Cu) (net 5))
 (segment (start 163.1 125.5) (end 163.5 125.9) (width 0.15) (layer B.Cu) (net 5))
 (segment (start 163.5 125.9) (end 163.5 125.9) (width 0.15) (layer B.Cu) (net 5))
 (via (at 163.5 125.9) (size 0.4) (drill 0.2) (layers F.Cu B.Cu) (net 5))
 (segment (start 173.931188 125.9) (end 173.957727 125.873461) (width 0.15) (layer F.Cu) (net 5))
 (segment (start 163.5 125.9) (end 173.931188 125.9) (width 0.15) (layer F.Cu) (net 5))
 (segment (start 147.372601 118.792641) (end 162.407359 118.792641) (width 0.15) (layer F.Cu) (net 4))
 (segment (start 162.407359 118.792641) (end 163.1 118.1) (width 0.15) (layer F.Cu) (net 4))
 (segment (start 163.1 118.1) (end 163.1 118.1) (width 0.15) (layer F.Cu) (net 4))
 (via (at 163.1 118.1) (size 0.4) (drill 0.2) (layers F.Cu B.Cu) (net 4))
 (segment (start 163.1 115.179099) (end 163.10645 115.172649) (width 0.15) (layer B.Cu) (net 4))
 (segment (start 163.1 118.1) (end 163.1 115.179099) (width 0.15) (layer B.Cu) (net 4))
 (segment (start 145.237562 117.416702) (end 147.716702 117.416702) (width 0.15) (layer F.Cu) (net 3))
 (segment (start 147.716702 117.416702) (end 148 117.7) (width 0.15) (layer F.Cu) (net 3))
 (segment (start 148 117.7) (end 148.3 118) (width 0.15) (layer F.Cu) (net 3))
 (segment (start 148.3 118) (end 151.1 118) (width 0.15) (layer F.Cu) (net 3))
 (segment (start 151.1 118) (end 151.4 118.3) (width 0.15) (layer F.Cu) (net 3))
 (segment (start 151.4 118.3) (end 151.4 118.3) (width 0.15) (layer F.Cu) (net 3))
 (via (at 151.4 118.3) (size 0.4) (drill 0.2) (layers F.Cu B.Cu) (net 3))
 (segment (start 168.9 141.1) (end 162.5 141.1) (width 0.15) (layer F.Cu) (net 3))
 (segment (start 162.5 141.1) (end 161.2 141.1) (width 0.15) (layer F.Cu) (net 3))
 (segment (start 161.2 141.1) (end 152.1 141.1) (width 0.15) (layer F.Cu) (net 3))
 (segment (start 152.1 141.1) (end 151.4 141.8) (width 0.15) (layer F.Cu) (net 3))
 (segment (start 151.4 141.8) (end 151.4 141.8) (width 0.15) (layer F.Cu) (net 3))
 (via (at 151.4 141.8) (size 0.4) (drill 0.2) (layers F.Cu B.Cu) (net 3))
 (segment (start 151.4 118.3) (end 151.4094 149.479) (width 0.15) (layer B.Cu) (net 3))
 (segment (start 151.8826 149.9522) (end 151.4094 149.479) (width 0.15) (layer B.Cu) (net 3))
 (segment (start 154.3 149.9522) (end 151.8826 149.9522) (width 0.15) (layer B.Cu) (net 3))
 (segment (start 164.61648 116.657602) (end 164.914996 116.956118) (width 0.15) (layer F.Cu) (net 2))
 (segment (start 148.74854 116.657602) (end 164.61648 116.657602) (width 0.15) (layer F.Cu) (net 2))
 (segment (start 175.766273 127.65693) (end 154.25693 127.65693) (width 0.6) (layer F.Cu) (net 1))
 (segment (start 154.25693 127.65693) (end 153.4 126.8) (width 0.6) (layer F.Cu) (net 1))
 (segment (start 153.4 126.8) (end 153.4 126.8) (width 0.6) (layer F.Cu) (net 1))
 (via (at 153.4 126.8) (size 0.6) (drill 0.3) (layers F.Cu B.Cu) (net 1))
 (segment (start 146.613501 115.281663) (end 147.595164 114.3) (width 0.6) (layer F.Cu) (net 1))
 (segment (start 147.595164 114.3) (end 149.86 114.3) (width 0.6) (layer F.Cu) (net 1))
 (segment (start 149.86 114.3) (end 149.86 114.3) (width 0.6) (layer F.Cu) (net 1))
 (via (at 151.13 114.3) (size 0.6) (drill 0.3) (layers F.Cu B.Cu) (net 1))
 (segment (start 153.4 116.57) (end 151.13 114.3) (width 0.6) (layer B.Cu) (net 1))
 (segment (start 153.4 126.8) (end 153.4 116.57) (width 0.6) (layer B.Cu) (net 1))
 (segment (start 149.86 114.3) (end 151.13 114.3) (width 0.6) (layer F.Cu) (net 1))
 (segment (start 153.072286 132.391191) (end 152.559286 131.878191) (width 0.15) (layer F.Cu) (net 19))
 (segment (start 156.959285 132.391191) (end 153.072286 132.391191) (width 0.15) (layer F.Cu) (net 19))
 (segment (start 153.046286 133.791191) (end 152.559286 134.278191) (width 0.15) (layer F.Cu) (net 17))
 (segment (start 156.959285 133.791191) (end 153.046286 133.791191) (width 0.15) (layer F.Cu) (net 17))
 (segment (start 164.946287 133.791191) (end 164.959286 133.778192) (width 0.15) (layer F.Cu) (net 18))
 (segment (start 159.459285 133.791191) (end 164.946287 133.791191) (width 0.15) (layer F.Cu) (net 18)))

